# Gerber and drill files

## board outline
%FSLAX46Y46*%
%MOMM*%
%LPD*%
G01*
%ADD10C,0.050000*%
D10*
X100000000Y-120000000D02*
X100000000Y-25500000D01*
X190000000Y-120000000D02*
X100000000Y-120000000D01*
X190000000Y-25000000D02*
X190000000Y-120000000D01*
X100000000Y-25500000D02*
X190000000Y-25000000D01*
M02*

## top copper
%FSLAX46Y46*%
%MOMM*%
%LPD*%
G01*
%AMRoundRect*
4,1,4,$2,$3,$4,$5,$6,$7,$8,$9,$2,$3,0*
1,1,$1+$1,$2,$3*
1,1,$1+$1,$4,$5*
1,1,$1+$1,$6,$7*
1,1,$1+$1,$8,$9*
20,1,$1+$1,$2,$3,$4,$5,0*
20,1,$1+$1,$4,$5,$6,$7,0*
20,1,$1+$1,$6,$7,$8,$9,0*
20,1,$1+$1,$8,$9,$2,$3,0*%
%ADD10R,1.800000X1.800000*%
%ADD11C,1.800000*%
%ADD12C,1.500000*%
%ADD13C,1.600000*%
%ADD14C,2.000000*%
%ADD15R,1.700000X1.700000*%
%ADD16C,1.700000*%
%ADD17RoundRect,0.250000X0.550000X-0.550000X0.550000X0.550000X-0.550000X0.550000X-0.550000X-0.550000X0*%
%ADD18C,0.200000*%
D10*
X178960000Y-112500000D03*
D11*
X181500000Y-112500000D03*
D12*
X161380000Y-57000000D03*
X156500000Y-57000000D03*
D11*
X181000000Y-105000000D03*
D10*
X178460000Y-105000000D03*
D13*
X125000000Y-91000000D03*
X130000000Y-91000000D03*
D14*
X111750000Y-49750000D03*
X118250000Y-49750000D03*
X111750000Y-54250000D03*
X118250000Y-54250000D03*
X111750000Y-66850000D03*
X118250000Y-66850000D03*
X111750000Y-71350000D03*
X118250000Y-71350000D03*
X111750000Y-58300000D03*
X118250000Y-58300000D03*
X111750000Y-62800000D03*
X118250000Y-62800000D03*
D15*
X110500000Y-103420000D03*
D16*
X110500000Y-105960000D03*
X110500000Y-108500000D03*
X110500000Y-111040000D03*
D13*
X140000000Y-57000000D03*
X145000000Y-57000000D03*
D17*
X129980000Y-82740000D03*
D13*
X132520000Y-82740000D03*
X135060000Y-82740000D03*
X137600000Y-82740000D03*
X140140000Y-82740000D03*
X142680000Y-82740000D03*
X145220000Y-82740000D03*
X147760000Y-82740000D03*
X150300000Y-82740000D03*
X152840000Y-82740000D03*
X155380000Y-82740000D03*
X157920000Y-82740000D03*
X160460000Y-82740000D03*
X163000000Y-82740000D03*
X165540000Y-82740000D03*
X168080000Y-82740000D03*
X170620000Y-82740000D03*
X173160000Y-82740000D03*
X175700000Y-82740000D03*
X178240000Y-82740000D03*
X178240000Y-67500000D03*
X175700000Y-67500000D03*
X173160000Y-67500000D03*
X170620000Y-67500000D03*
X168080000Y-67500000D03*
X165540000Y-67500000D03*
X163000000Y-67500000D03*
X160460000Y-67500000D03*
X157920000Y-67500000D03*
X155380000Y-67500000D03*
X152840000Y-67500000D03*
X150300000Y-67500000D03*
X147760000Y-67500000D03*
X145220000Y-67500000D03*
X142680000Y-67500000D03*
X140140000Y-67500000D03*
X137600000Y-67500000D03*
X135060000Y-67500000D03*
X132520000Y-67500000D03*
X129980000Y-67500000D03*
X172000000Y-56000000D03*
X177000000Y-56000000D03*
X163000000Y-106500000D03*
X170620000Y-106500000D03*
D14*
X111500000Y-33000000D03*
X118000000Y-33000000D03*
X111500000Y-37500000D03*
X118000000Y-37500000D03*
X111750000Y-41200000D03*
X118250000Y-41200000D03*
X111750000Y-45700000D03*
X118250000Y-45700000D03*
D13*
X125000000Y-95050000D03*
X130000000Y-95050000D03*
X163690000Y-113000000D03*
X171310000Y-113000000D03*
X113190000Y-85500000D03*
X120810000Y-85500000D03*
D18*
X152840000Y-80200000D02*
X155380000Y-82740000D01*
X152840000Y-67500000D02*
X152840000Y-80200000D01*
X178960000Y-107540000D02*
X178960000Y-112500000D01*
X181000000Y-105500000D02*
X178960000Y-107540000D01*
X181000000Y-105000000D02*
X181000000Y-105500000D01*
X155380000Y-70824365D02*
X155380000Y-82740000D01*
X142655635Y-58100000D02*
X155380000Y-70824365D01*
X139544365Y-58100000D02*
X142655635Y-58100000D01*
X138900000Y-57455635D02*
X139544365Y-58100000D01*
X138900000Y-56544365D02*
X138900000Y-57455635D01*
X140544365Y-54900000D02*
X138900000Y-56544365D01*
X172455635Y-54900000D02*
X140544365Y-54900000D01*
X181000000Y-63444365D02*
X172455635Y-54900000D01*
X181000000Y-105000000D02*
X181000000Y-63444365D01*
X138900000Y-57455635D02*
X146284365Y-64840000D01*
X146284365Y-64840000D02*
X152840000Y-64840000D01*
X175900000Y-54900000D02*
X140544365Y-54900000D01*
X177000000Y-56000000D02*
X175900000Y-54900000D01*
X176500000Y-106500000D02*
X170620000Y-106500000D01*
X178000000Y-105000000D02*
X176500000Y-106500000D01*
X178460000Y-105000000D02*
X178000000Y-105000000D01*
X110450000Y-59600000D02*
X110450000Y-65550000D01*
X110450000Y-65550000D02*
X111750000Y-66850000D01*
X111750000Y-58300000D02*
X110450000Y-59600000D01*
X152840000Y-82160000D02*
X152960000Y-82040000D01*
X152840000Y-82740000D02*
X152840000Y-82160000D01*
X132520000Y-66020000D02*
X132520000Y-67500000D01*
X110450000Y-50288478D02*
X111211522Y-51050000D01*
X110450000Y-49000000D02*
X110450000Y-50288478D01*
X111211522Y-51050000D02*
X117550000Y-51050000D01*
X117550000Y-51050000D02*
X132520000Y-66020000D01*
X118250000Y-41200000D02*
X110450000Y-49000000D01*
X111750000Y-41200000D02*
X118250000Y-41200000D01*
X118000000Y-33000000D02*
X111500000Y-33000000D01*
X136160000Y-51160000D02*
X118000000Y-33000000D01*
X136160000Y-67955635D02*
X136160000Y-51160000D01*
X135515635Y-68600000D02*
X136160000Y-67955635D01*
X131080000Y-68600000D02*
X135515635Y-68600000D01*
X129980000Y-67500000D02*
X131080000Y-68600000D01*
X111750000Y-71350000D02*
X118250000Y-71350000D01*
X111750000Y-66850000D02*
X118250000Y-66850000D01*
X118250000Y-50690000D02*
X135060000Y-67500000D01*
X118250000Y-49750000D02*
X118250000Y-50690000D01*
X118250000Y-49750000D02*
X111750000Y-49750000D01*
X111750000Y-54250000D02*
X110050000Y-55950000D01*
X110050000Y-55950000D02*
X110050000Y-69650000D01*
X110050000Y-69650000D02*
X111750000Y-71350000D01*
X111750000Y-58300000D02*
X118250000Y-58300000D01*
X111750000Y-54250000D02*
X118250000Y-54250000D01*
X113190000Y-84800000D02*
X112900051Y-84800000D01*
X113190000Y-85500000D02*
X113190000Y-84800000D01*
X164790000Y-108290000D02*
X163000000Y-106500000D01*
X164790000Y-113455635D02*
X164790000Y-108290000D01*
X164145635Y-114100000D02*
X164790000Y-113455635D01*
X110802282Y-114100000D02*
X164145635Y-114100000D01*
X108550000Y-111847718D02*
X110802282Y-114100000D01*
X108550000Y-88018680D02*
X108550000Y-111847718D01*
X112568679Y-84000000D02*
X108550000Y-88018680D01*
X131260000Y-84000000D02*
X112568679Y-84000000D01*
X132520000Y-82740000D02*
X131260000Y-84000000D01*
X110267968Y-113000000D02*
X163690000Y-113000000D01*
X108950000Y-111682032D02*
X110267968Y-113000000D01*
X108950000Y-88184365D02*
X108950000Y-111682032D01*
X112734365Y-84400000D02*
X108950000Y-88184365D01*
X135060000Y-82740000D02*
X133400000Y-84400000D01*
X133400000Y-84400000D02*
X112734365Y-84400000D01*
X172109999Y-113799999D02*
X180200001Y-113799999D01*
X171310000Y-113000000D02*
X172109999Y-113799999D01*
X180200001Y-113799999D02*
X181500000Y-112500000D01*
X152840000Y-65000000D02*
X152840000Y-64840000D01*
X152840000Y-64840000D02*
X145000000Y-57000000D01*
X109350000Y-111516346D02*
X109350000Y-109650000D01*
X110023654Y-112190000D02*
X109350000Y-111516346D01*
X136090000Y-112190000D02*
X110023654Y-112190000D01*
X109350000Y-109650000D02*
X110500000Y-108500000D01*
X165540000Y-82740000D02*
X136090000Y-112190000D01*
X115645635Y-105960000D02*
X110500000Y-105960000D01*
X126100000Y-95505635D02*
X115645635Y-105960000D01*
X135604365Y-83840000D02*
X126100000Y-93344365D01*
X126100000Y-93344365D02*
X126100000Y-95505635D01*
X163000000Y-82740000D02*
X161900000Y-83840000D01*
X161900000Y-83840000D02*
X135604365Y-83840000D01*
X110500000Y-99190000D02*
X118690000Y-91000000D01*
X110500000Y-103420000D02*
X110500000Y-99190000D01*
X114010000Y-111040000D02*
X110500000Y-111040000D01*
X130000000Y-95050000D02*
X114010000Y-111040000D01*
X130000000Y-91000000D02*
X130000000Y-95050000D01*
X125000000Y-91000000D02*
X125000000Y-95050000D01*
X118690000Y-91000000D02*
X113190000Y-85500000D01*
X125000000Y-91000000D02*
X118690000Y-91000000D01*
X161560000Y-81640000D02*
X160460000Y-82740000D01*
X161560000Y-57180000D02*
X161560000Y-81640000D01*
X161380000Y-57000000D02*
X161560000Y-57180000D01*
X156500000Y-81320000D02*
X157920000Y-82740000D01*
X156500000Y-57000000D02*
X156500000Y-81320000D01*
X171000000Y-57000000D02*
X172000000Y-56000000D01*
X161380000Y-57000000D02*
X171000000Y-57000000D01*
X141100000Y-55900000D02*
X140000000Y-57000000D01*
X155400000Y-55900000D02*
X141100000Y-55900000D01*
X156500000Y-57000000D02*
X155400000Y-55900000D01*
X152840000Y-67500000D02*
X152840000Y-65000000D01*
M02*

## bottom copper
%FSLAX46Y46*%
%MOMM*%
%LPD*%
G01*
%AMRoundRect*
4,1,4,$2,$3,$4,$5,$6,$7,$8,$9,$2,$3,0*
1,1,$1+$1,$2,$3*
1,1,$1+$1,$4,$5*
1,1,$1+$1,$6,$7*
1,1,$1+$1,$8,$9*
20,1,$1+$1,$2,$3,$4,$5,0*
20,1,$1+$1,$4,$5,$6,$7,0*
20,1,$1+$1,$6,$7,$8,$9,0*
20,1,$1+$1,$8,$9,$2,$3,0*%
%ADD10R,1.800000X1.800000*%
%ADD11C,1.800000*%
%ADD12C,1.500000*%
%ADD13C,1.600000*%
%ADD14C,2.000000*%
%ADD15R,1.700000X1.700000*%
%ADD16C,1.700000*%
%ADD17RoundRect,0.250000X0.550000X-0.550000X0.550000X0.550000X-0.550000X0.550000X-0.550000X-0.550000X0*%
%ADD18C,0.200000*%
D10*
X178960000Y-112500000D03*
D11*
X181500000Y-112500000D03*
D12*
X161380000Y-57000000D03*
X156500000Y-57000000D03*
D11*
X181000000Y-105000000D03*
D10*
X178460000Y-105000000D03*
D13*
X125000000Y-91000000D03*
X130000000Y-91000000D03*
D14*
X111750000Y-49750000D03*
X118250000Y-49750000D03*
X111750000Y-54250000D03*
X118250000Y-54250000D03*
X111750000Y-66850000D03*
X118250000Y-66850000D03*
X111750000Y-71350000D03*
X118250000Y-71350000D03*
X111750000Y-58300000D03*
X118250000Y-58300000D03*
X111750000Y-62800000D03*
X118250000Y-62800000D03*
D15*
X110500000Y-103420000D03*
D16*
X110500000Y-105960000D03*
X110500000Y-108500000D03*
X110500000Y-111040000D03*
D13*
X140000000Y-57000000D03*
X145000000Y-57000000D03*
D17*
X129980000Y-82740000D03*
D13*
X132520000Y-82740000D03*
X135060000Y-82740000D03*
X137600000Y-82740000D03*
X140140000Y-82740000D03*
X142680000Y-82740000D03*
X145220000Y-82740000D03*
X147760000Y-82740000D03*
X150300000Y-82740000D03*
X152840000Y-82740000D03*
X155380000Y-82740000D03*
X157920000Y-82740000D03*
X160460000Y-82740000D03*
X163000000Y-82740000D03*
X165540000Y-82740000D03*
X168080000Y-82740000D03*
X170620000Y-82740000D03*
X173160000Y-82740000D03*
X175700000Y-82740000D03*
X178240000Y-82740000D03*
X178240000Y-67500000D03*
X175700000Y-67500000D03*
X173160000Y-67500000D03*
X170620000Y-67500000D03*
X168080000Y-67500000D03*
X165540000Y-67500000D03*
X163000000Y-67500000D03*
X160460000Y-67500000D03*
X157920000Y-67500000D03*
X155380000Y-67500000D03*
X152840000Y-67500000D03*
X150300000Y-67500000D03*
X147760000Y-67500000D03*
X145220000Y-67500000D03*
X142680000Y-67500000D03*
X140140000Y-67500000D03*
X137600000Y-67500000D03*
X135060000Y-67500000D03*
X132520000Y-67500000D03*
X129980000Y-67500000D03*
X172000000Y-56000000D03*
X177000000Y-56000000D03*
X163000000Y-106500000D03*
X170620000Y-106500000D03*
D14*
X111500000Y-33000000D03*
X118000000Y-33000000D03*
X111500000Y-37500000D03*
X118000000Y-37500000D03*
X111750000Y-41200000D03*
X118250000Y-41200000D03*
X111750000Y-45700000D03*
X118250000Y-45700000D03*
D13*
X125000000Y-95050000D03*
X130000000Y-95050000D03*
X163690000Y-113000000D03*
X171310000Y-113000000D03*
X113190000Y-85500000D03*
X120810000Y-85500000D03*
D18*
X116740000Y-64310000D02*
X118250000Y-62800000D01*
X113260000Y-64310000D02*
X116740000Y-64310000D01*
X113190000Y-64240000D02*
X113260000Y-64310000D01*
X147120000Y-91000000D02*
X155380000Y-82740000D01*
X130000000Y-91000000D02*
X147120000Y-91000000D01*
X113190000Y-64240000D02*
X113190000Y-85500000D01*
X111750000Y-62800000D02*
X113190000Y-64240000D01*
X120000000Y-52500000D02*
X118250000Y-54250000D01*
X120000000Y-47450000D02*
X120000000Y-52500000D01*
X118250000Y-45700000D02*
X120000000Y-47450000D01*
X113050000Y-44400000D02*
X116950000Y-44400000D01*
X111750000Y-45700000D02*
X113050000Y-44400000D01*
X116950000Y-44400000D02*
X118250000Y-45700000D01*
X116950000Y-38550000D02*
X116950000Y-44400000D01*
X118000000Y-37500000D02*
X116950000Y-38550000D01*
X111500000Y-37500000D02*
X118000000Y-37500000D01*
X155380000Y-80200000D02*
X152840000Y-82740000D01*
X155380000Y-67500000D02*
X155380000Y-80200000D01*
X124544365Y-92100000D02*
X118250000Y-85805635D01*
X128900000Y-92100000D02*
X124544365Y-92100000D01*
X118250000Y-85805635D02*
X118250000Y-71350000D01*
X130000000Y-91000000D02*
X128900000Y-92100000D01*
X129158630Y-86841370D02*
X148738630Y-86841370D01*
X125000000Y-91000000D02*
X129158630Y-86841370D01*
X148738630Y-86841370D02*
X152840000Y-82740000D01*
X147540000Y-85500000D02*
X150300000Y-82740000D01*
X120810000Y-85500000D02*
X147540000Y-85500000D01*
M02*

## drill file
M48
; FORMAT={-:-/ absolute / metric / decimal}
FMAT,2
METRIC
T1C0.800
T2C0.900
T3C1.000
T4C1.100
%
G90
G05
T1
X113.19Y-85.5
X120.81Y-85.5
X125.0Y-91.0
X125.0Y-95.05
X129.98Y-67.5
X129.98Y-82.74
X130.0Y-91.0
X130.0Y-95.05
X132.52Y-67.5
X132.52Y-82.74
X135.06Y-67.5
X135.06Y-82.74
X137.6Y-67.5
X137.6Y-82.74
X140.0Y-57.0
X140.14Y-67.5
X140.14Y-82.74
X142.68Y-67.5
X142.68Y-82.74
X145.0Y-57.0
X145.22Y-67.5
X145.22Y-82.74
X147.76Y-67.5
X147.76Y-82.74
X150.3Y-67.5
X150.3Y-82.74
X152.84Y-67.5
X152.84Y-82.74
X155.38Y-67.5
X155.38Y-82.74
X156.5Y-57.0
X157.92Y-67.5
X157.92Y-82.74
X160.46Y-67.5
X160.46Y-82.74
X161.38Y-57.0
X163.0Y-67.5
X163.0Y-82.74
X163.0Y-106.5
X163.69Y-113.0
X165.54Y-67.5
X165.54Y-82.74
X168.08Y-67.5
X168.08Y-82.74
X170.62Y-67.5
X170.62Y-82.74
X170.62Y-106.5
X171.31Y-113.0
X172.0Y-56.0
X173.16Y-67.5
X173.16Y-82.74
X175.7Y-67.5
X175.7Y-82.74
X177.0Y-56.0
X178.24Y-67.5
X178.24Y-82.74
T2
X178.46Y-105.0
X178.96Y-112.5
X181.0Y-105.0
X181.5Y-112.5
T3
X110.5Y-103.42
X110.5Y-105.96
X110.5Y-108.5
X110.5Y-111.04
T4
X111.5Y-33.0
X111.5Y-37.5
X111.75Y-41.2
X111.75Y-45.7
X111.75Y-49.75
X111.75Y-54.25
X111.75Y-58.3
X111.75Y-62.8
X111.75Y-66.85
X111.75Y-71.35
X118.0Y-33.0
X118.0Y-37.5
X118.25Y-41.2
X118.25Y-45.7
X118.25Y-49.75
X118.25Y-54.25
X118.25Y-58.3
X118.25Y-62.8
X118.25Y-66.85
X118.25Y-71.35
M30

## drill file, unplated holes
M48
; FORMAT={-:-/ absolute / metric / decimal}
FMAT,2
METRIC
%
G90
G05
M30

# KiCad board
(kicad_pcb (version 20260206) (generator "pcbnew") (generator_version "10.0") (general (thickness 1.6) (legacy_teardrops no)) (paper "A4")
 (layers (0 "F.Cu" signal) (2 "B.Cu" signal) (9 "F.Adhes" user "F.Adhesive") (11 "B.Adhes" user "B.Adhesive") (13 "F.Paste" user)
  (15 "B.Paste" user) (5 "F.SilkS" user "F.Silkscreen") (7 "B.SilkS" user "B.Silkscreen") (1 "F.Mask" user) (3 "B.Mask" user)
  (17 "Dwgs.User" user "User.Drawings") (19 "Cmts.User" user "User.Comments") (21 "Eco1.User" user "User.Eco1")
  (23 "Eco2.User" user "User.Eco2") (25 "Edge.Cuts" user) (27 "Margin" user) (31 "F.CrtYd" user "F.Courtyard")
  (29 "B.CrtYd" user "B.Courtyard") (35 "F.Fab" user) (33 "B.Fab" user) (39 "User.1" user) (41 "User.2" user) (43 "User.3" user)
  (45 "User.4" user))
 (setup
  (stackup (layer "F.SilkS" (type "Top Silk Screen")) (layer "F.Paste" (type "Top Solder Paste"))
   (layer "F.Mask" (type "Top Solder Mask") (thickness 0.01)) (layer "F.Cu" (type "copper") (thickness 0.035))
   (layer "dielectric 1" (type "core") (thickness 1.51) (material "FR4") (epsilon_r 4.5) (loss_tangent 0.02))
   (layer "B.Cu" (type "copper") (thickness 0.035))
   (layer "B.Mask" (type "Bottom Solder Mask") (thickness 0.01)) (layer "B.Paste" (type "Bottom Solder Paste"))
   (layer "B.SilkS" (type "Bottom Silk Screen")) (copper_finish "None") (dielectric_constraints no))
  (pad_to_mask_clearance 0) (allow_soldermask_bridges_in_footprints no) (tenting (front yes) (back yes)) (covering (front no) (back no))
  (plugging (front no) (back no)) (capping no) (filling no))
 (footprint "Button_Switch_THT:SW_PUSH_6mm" (layer "F.Cu") (at 111.75 49.75)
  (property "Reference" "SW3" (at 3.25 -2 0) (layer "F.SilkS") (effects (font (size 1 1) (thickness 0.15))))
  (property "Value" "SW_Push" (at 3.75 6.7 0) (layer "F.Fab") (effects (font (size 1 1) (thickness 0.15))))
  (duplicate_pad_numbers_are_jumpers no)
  (pad "1" thru_hole circle (at 0 0 90) (size 2 2) (drill 1.1) (layers "*.Cu" "*.Mask") (remove_unused_layers no) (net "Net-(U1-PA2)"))
  (pad "1" thru_hole circle (at 6.5 0 90) (size 2 2) (drill 1.1) (layers "*.Cu" "*.Mask") (remove_unused_layers no) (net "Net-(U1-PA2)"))
  (pad "2" thru_hole circle (at 0 4.5 90) (size 2 2) (drill 1.1) (layers "*.Cu" "*.Mask") (remove_unused_layers no) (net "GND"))
  (pad "2" thru_hole circle (at 6.5 4.5 90) (size 2 2) (drill 1.1) (layers "*.Cu" "*.Mask") (remove_unused_layers no) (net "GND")))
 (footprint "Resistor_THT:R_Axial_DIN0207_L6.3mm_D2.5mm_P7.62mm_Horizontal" (layer "F.Cu") (at 113.19 85.5)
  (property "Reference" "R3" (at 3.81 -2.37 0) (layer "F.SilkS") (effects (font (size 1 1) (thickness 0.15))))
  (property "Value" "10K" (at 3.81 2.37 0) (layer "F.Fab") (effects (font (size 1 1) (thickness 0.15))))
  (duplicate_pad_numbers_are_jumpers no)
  (pad "1" thru_hole circle (at 0 0) (size 1.6 1.6) (drill 0.8) (layers "*.Cu" "*.Mask") (remove_unused_layers no) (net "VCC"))
  (pad "2" thru_hole circle (at 7.62 0) (size 1.6 1.6) (drill 0.8) (layers "*.Cu" "*.Mask") (remove_unused_layers no)
   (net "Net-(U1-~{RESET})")))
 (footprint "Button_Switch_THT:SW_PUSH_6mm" (layer "F.Cu") (at 111.75 41.2)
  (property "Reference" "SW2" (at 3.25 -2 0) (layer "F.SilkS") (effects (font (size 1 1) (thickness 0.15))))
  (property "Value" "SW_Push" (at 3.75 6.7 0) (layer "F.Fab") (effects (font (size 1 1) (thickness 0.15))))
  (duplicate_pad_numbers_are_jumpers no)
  (pad "1" thru_hole circle (at 0 0 90) (size 2 2) (drill 1.1) (layers "*.Cu" "*.Mask") (remove_unused_layers no) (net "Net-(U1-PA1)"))
  (pad "1" thru_hole circle (at 6.5 0 90) (size 2 2) (drill 1.1) (layers "*.Cu" "*.Mask") (remove_unused_layers no) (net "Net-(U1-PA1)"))
  (pad "2" thru_hole circle (at 0 4.5 90) (size 2 2) (drill 1.1) (layers "*.Cu" "*.Mask") (remove_unused_layers no) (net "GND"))
  (pad "2" thru_hole circle (at 6.5 4.5 90) (size 2 2) (drill 1.1) (layers "*.Cu" "*.Mask") (remove_unused_layers no) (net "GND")))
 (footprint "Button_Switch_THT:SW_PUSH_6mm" (layer "F.Cu") (at 111.75 66.85)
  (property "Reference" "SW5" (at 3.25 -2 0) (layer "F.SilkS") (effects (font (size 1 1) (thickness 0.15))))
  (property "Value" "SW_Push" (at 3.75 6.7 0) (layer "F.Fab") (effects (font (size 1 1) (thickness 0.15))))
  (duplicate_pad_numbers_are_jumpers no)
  (pad "1" thru_hole circle (at 0 0 90) (size 2 2) (drill 1.1) (layers "*.Cu" "*.Mask") (remove_unused_layers no) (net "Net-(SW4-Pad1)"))
  (pad "1" thru_hole circle (at 6.5 0 90) (size 2 2) (drill 1.1) (layers "*.Cu" "*.Mask") (remove_unused_layers no) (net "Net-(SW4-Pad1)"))
  (pad "2" thru_hole circle (at 0 4.5 90) (size 2 2) (drill 1.1) (layers "*.Cu" "*.Mask") (remove_unused_layers no) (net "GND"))
  (pad "2" thru_hole circle (at 6.5 4.5 90) (size 2 2) (drill 1.1) (layers "*.Cu" "*.Mask") (remove_unused_layers no) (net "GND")))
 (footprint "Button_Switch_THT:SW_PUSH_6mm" (layer "F.Cu") (at 111.5 33)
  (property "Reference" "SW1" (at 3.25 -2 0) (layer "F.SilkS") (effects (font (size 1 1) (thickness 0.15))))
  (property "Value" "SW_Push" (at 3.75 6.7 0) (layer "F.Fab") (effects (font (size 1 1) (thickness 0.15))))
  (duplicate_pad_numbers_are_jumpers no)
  (pad "1" thru_hole circle (at 0 0 90) (size 2 2) (drill 1.1) (layers "*.Cu" "*.Mask") (remove_unused_layers no) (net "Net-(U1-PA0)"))
  (pad "1" thru_hole circle (at 6.5 0 90) (size 2 2) (drill 1.1) (layers "*.Cu" "*.Mask") (remove_unused_layers no) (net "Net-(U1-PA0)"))
  (pad "2" thru_hole circle (at 0 4.5 90) (size 2 2) (drill 1.1) (layers "*.Cu" "*.Mask") (remove_unused_layers no) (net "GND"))
  (pad "2" thru_hole circle (at 6.5 4.5 90) (size 2 2) (drill 1.1) (layers "*.Cu" "*.Mask") (remove_unused_layers no) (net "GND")))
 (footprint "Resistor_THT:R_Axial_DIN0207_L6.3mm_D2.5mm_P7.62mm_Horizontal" (layer "F.Cu") (at 163.69 113)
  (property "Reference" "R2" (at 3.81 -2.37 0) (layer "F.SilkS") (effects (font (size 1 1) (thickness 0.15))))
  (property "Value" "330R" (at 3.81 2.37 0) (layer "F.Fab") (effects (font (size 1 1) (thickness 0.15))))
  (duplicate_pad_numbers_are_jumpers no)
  (pad "1" thru_hole circle (at 0 0) (size 1.6 1.6) (drill 0.8) (layers "*.Cu" "*.Mask") (remove_unused_layers no) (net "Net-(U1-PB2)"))
  (pad "2" thru_hole circle (at 7.62 0) (size 1.6 1.6) (drill 0.8) (layers "*.Cu" "*.Mask") (remove_unused_layers no) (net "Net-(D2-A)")))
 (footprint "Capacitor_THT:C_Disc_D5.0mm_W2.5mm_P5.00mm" (layer "F.Cu") (at 125 95.05)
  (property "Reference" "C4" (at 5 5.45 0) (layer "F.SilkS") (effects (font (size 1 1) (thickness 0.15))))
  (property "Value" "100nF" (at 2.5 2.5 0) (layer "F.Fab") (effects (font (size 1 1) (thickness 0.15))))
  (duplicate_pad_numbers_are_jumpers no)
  (pad "1" thru_hole circle (at 0 0) (size 1.6 1.6) (drill 0.8) (layers "*.Cu" "*.Mask") (remove_unused_layers no) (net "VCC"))
  (pad "2" thru_hole circle (at 5 0) (size 1.6 1.6) (drill 0.8) (layers "*.Cu" "*.Mask") (remove_unused_layers no) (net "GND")))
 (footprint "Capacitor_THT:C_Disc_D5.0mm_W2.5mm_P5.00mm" (layer "F.Cu") (at 172 56)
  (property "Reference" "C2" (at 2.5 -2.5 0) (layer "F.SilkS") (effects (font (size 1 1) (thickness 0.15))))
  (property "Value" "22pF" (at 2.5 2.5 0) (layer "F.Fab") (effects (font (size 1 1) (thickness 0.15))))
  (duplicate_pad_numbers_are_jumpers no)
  (pad "1" thru_hole circle (at 0 0) (size 1.6 1.6) (drill 0.8) (layers "*.Cu" "*.Mask") (remove_unused_layers no) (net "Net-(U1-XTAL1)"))
  (pad "2" thru_hole circle (at 5 0) (size 1.6 1.6) (drill 0.8) (layers "*.Cu" "*.Mask") (remove_unused_layers no) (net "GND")))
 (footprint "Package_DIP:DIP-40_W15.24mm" (layer "F.Cu") (at 129.98 82.74 90)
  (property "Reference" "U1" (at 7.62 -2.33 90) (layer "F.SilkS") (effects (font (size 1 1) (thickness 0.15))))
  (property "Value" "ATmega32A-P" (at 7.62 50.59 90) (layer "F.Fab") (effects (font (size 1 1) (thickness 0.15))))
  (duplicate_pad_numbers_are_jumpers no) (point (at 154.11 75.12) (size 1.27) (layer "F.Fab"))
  (pad "1" thru_hole roundrect (at 0 0 90) (size 1.6 1.6) (drill 0.8) (layers "*.Cu" "*.Mask") (remove_unused_layers no)
   (roundrect_rratio 0.15625) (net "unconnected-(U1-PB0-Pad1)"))
  (pad "2" thru_hole circle (at 0 2.54 90) (size 1.6 1.6) (drill 0.8) (layers "*.Cu" "*.Mask") (remove_unused_layers no)
   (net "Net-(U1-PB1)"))
  (pad "3" thru_hole circle (at 0 5.08 90) (size 1.6 1.6) (drill 0.8) (layers "*.Cu" "*.Mask") (remove_unused_layers no)
   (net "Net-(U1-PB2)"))
  (pad "4" thru_hole circle (at 0 7.62 90) (size 1.6 1.6) (drill 0.8) (layers "*.Cu" "*.Mask") (remove_unused_layers no)
   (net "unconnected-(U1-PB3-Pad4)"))
  (pad "5" thru_hole circle (at 0 10.16 90) (size 1.6 1.6) (drill 0.8) (layers "*.Cu" "*.Mask") (remove_unused_layers no)
   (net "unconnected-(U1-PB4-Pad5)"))
  (pad "6" thru_hole circle (at 0 12.7 90) (size 1.6 1.6) (drill 0.8) (layers "*.Cu" "*.Mask") (remove_unused_layers no)
   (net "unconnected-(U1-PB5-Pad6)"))
  (pad "7" thru_hole circle (at 0 15.24 90) (size 1.6 1.6) (drill 0.8) (layers "*.Cu" "*.Mask") (remove_unused_layers no)
   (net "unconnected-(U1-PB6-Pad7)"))
  (pad "8" thru_hole circle (at 0 17.78 90) (size 1.6 1.6) (drill 0.8) (layers "*.Cu" "*.Mask") (remove_unused_layers no)
   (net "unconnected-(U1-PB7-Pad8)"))
  (pad "9" thru_hole circle (at 0 20.32 90) (size 1.6 1.6) (drill 0.8) (layers "*.Cu" "*.Mask") (remove_unused_layers no)
   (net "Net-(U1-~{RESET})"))
  (pad "10" thru_hole circle (at 0 22.86 90) (size 1.6 1.6) (drill 0.8) (layers "*.Cu" "*.Mask") (remove_unused_layers no) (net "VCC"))
  (pad "11" thru_hole circle (at 0 25.4 90) (size 1.6 1.6) (drill 0.8) (layers "*.Cu" "*.Mask") (remove_unused_layers no) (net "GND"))
  (pad "12" thru_hole circle (at 0 27.94 90) (size 1.6 1.6) (drill 0.8) (layers "*.Cu" "*.Mask") (remove_unused_layers no)
   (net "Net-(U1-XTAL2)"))
  (pad "13" thru_hole circle (at 0 30.48 90) (size 1.6 1.6) (drill 0.8) (layers "*.Cu" "*.Mask") (remove_unused_layers no)
   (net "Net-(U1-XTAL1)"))
  (pad "14" thru_hole circle (at 0 33.02 90) (size 1.6 1.6) (drill 0.8) (layers "*.Cu" "*.Mask") (remove_unused_layers no)
   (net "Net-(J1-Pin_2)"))
  (pad "15" thru_hole circle (at 0 35.56 90) (size 1.6 1.6) (drill 0.8) (layers "*.Cu" "*.Mask") (remove_unused_layers no)
   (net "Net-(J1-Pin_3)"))
  (pad "16" thru_hole circle (at 0 38.1 90) (size 1.6 1.6) (drill 0.8) (layers "*.Cu" "*.Mask") (remove_unused_layers no)
   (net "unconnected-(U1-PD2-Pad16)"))
  (pad "17" thru_hole circle (at 0 40.64 90) (size 1.6 1.6) (drill 0.8) (layers "*.Cu" "*.Mask") (remove_unused_layers no)
   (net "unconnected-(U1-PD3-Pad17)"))
  (pad "18" thru_hole circle (at 0 43.18 90) (size 1.6 1.6) (drill 0.8) (layers "*.Cu" "*.Mask") (remove_unused_layers no)
   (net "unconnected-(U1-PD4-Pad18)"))
  (pad "19" thru_hole circle (at 0 45.72 90) (size 1.6 1.6) (drill 0.8) (layers "*.Cu" "*.Mask") (remove_unused_layers no)
   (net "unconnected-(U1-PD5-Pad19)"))
  (pad "20" thru_hole circle (at 0 48.26 90) (size 1.6 1.6) (drill 0.8) (layers "*.Cu" "*.Mask") (remove_unused_layers no)
   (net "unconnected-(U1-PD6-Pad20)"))
  (pad "21" thru_hole circle (at 15.24 48.26 90) (size 1.6 1.6) (drill 0.8) (layers "*.Cu" "*.Mask") (remove_unused_layers no)
   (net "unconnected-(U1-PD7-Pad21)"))
  (pad "22" thru_hole circle (at 15.24 45.72 90) (size 1.6 1.6) (drill 0.8) (layers "*.Cu" "*.Mask") (remove_unused_layers no)
   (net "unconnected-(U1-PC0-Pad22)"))
  (pad "23" thru_hole circle (at 15.24 43.18 90) (size 1.6 1.6) (drill 0.8) (layers "*.Cu" "*.Mask") (remove_unused_layers no)
   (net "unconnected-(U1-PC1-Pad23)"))
  (pad "24" thru_hole circle (at 15.24 40.64 90) (size 1.6 1.6) (drill 0.8) (layers "*.Cu" "*.Mask") (remove_unused_layers no)
   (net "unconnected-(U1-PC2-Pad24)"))
  (pad "25" thru_hole circle (at 15.24 38.1 90) (size 1.6 1.6) (drill 0.8) (layers "*.Cu" "*.Mask") (remove_unused_layers no)
   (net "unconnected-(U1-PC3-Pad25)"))
  (pad "26" thru_hole circle (at 15.24 35.56 90) (size 1.6 1.6) (drill 0.8) (layers "*.Cu" "*.Mask") (remove_unused_layers no)
   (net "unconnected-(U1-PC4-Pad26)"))
  (pad "27" thru_hole circle (at 15.24 33.02 90) (size 1.6 1.6) (drill 0.8) (layers "*.Cu" "*.Mask") (remove_unused_layers no)
   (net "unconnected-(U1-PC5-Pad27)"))
  (pad "28" thru_hole circle (at 15.24 30.48 90) (size 1.6 1.6) (drill 0.8) (layers "*.Cu" "*.Mask") (remove_unused_layers no)
   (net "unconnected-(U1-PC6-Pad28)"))
  (pad "29" thru_hole circle (at 15.24 27.94 90) (size 1.6 1.6) (drill 0.8) (layers "*.Cu" "*.Mask") (remove_unused_layers no)
   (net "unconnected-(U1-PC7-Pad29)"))
  (pad "30" thru_hole circle (at 15.24 25.4 90) (size 1.6 1.6) (drill 0.8) (layers "*.Cu" "*.Mask") (remove_unused_layers no) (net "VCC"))
  (pad "31" thru_hole circle (at 15.24 22.86 90) (size 1.6 1.6) (drill 0.8) (layers "*.Cu" "*.Mask") (remove_unused_layers no) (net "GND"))
  (pad "32" thru_hole circle (at 15.24 20.32 90) (size 1.6 1.6) (drill 0.8) (layers "*.Cu" "*.Mask") (remove_unused_layers no)
   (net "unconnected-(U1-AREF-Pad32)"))
  (pad "33" thru_hole circle (at 15.24 17.78 90) (size 1.6 1.6) (drill 0.8) (layers "*.Cu" "*.Mask") (remove_unused_layers no)
   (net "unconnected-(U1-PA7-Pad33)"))
  (pad "34" thru_hole circle (at 15.24 15.24 90) (size 1.6 1.6) (drill 0.8) (layers "*.Cu" "*.Mask") (remove_unused_layers no)
   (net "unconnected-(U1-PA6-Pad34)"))
  (pad "35" thru_hole circle (at 15.24 12.7 90) (size 1.6 1.6) (drill 0.8) (layers "*.Cu" "*.Mask") (remove_unused_layers no)
   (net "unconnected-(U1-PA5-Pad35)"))
  (pad "36" thru_hole circle (at 15.24 10.16 90) (size 1.6 1.6) (drill 0.8) (layers "*.Cu" "*.Mask") (remove_unused_layers no)
   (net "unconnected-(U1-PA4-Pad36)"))
  (pad "37" thru_hole circle (at 15.24 7.62 90) (size 1.6 1.6) (drill 0.8) (layers "*.Cu" "*.Mask") (remove_unused_layers no)
   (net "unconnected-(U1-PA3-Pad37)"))
  (pad "38" thru_hole circle (at 15.24 5.08 90) (size 1.6 1.6) (drill 0.8) (layers "*.Cu" "*.Mask") (remove_unused_layers no)
   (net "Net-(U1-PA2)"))
  (pad "39" thru_hole circle (at 15.24 2.54 90) (size 1.6 1.6) (drill 0.8) (layers "*.Cu" "*.Mask") (remove_unused_layers no)
   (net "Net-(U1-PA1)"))
  (pad "40" thru_hole circle (at 15.24 0 90) (size 1.6 1.6) (drill 0.8) (layers "*.Cu" "*.Mask") (remove_unused_layers no)
   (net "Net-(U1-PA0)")))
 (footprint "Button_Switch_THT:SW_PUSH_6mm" (layer "F.Cu") (at 111.75 58.3)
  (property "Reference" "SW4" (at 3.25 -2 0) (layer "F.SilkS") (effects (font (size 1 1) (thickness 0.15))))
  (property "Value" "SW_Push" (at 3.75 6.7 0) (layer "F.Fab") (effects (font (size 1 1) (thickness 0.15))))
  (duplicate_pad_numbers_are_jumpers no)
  (pad "1" thru_hole circle (at 0 0 90) (size 2 2) (drill 1.1) (layers "*.Cu" "*.Mask") (remove_unused_layers no) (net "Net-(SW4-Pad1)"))
  (pad "1" thru_hole circle (at 6.5 0 90) (size 2 2) (drill 1.1) (layers "*.Cu" "*.Mask") (remove_unused_layers no) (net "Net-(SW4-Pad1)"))
  (pad "2" thru_hole circle (at 0 4.5 90) (size 2 2) (drill 1.1) (layers "*.Cu" "*.Mask") (remove_unused_layers no) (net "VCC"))
  (pad "2" thru_hole circle (at 6.5 4.5 90) (size 2 2) (drill 1.1) (layers "*.Cu" "*.Mask") (remove_unused_layers no) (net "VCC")))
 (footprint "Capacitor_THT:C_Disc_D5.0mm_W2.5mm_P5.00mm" (layer "F.Cu") (at 125 91)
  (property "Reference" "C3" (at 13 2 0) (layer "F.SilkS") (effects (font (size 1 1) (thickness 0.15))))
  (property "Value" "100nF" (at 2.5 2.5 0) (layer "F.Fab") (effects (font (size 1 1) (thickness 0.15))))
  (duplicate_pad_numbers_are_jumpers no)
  (pad "1" thru_hole circle (at 0 0) (size 1.6 1.6) (drill 0.8) (layers "*.Cu" "*.Mask") (remove_unused_layers no) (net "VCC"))
  (pad "2" thru_hole circle (at 5 0) (size 1.6 1.6) (drill 0.8) (layers "*.Cu" "*.Mask") (remove_unused_layers no) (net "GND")))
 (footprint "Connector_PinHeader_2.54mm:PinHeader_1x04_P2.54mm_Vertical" (layer "F.Cu") (at 110.5 103.42)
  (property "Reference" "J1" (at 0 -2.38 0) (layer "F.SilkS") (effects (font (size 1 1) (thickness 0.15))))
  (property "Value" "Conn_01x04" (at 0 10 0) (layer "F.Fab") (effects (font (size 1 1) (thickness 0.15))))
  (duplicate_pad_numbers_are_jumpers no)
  (pad "1" thru_hole rect (at 0 0) (size 1.7 1.7) (drill 1) (layers "*.Cu" "*.Mask") (remove_unused_layers no) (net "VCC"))
  (pad "2" thru_hole circle (at 0 2.54) (size 1.7 1.7) (drill 1) (layers "*.Cu" "*.Mask") (remove_unused_layers no) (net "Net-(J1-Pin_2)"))
  (pad "3" thru_hole circle (at 0 5.08) (size 1.7 1.7) (drill 1) (layers "*.Cu" "*.Mask") (remove_unused_layers no) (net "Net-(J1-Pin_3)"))
  (pad "4" thru_hole circle (at 0 7.62) (size 1.7 1.7) (drill 1) (layers "*.Cu" "*.Mask") (remove_unused_layers no) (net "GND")))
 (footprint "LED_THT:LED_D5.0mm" (layer "F.Cu") (at 178.96 112.5)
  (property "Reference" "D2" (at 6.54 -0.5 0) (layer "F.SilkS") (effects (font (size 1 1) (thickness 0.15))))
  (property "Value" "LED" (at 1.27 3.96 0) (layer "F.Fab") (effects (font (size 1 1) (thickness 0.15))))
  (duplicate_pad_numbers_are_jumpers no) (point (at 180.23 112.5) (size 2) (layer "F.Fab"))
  (pad "1" thru_hole rect (at 0 0) (size 1.8 1.8) (drill 0.9) (layers "*.Cu" "*.Mask") (remove_unused_layers no) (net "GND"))
  (pad "2" thru_hole circle (at 2.54 0) (size 1.8 1.8) (drill 0.9) (layers "*.Cu" "*.Mask") (remove_unused_layers no) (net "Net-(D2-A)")))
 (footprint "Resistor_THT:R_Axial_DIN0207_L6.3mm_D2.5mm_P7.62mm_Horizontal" (layer "F.Cu") (at 163 106.5)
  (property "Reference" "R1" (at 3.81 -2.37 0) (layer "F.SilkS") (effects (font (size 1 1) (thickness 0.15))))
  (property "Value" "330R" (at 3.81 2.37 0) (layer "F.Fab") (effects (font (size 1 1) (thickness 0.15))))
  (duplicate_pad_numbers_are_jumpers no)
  (pad "1" thru_hole circle (at 0 0) (size 1.6 1.6) (drill 0.8) (layers "*.Cu" "*.Mask") (remove_unused_layers no) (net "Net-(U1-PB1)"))
  (pad "2" thru_hole circle (at 7.62 0) (size 1.6 1.6) (drill 0.8) (layers "*.Cu" "*.Mask") (remove_unused_layers no) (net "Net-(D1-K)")))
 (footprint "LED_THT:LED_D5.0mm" (layer "F.Cu") (at 178.46 105)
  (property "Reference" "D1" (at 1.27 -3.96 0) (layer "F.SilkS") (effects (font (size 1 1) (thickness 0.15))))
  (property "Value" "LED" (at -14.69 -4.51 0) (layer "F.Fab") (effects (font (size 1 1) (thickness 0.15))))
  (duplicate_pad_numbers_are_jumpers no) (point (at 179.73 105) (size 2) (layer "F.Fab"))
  (pad "1" thru_hole rect (at 0 0) (size 1.8 1.8) (drill 0.9) (layers "*.Cu" "*.Mask") (remove_unused_layers no) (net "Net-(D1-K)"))
  (pad "2" thru_hole circle (at 2.54 0) (size 1.8 1.8) (drill 0.9) (layers "*.Cu" "*.Mask") (remove_unused_layers no) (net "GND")))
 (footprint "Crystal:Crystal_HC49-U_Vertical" (layer "F.Cu") (at 156.5 57)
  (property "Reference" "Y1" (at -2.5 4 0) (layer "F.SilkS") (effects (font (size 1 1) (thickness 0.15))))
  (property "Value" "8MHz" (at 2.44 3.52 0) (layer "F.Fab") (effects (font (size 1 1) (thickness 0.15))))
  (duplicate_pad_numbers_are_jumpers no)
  (pad "1" thru_hole circle (at 0 0) (size 1.5 1.5) (drill 0.8) (layers "*.Cu" "*.Mask") (remove_unused_layers no) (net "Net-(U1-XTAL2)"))
  (pad "2" thru_hole circle (at 4.88 0) (size 1.5 1.5) (drill 0.8) (layers "*.Cu" "*.Mask") (remove_unused_layers no) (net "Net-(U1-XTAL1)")))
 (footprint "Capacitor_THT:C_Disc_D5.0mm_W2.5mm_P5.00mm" (layer "F.Cu") (at 140 57)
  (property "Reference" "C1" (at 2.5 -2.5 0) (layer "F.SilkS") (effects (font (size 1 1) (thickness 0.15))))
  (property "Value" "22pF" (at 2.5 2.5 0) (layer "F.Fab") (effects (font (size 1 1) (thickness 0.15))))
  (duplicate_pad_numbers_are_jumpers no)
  (pad "1" thru_hole circle (at 0 0) (size 1.6 1.6) (drill 0.8) (layers "*.Cu" "*.Mask") (remove_unused_layers no) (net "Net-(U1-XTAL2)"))
  (pad "2" thru_hole circle (at 5 0) (size 1.6 1.6) (drill 0.8) (layers "*.Cu" "*.Mask") (remove_unused_layers no) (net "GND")))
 (gr_line (start 100 25.5) (end 190 25) (stroke (width 0.05) (type default)) (layer "Edge.Cuts"))
 (gr_line (start 100 120) (end 100 25.5) (stroke (width 0.05) (type default)) (layer "Edge.Cuts"))
 (gr_line (start 190 25) (end 190 120) (stroke (width 0.05) (type default)) (layer "Edge.Cuts"))
 (gr_line (start 190 120) (end 100 120) (stroke (width 0.05) (type default)) (layer "Edge.Cuts"))
 (segment (start 110.05 55.95) (end 110.05 69.65) (width 0.2) (layer "F.Cu") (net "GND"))
 (segment (start 181 105.5) (end 178.96 107.54) (width 0.2) (layer "F.Cu") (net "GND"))
 (segment (start 138.9 57.455635) (end 139.544365 58.1) (width 0.2) (layer "F.Cu") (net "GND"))
 (segment (start 142.655635 58.1) (end 155.38 70.824365) (width 0.2) (layer "F.Cu") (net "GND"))
 (segment (start 152.84 80.2) (end 155.38 82.74) (width 0.2) (layer "F.Cu") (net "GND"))
 (segment (start 138.9 57.455635) (end 146.284365 64.84) (width 0.2) (layer "F.Cu") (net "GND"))
 (segment (start 175.9 54.9) (end 140.544365 54.9) (width 0.2) (layer "F.Cu") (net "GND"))
 (segment (start 177 56) (end 175.9 54.9) (width 0.2) (layer "F.Cu") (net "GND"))
 (segment (start 152.84 65) (end 152.84 64.84) (width 0.2) (layer "F.Cu") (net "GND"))
 (segment (start 111.75 54.25) (end 118.25 54.25) (width 0.2) (layer "F.Cu") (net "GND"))
 (segment (start 152.84 67.5) (end 152.84 65) (width 0.2) (layer "F.Cu") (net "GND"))
 (segment (start 146.284365 64.84) (end 152.84 64.84) (width 0.2) (layer "F.Cu") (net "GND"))
 (segment (start 110.05 69.65) (end 111.75 71.35) (width 0.2) (layer "F.Cu") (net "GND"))
 (segment (start 152.84 64.84) (end 145 57) (width 0.2) (layer "F.Cu") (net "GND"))
 (segment (start 178.96 107.54) (end 178.96 112.5) (width 0.2) (layer "F.Cu") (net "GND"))
 (segment (start 140.544365 54.9) (end 138.9 56.544365) (width 0.2) (layer "F.Cu") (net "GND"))
 (segment (start 114.01 111.04) (end 110.5 111.04) (width 0.2) (layer "F.Cu") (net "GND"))
 (segment (start 138.9 56.544365) (end 138.9 57.455635) (width 0.2) (layer "F.Cu") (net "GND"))
 (segment (start 111.75 71.35) (end 118.25 71.35) (width 0.2) (layer "F.Cu") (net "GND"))
 (segment (start 181 105) (end 181 63.444365) (width 0.2) (layer "F.Cu") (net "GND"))
 (segment (start 181 105) (end 181 105.5) (width 0.2) (layer "F.Cu") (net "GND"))
 (segment (start 130 91) (end 130 95.05) (width 0.2) (layer "F.Cu") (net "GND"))
 (segment (start 172.455635 54.9) (end 140.544365 54.9) (width 0.2) (layer "F.Cu") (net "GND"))
 (segment (start 139.544365 58.1) (end 142.655635 58.1) (width 0.2) (layer "F.Cu") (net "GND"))
 (segment (start 155.38 70.824365) (end 155.38 82.74) (width 0.2) (layer "F.Cu") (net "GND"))
 (segment (start 130 95.05) (end 114.01 111.04) (width 0.2) (layer "F.Cu") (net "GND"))
 (segment (start 152.84 67.5) (end 152.84 80.2) (width 0.2) (layer "F.Cu") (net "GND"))
 (segment (start 181 63.444365) (end 172.455635 54.9) (width 0.2) (layer "F.Cu") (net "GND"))
 (segment (start 111.75 54.25) (end 110.05 55.95) (width 0.2) (layer "F.Cu") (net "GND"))
 (segment (start 120 47.45) (end 120 52.5) (width 0.2) (layer "B.Cu") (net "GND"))
 (segment (start 111.75 45.7) (end 113.05 44.4) (width 0.2) (layer "B.Cu") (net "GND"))
 (segment (start 113.05 44.4) (end 116.95 44.4) (width 0.2) (layer "B.Cu") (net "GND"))
 (segment (start 111.5 37.5) (end 118 37.5) (width 0.2) (layer "B.Cu") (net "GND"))
 (segment (start 124.544365 92.1) (end 118.25 85.805635) (width 0.2) (layer "B.Cu") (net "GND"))
 (segment (start 120 52.5) (end 118.25 54.25) (width 0.2) (layer "B.Cu") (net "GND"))
 (segment (start 118.25 85.805635) (end 118.25 71.35) (width 0.2) (layer "B.Cu") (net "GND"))
 (segment (start 116.95 44.4) (end 118.25 45.7) (width 0.2) (layer "B.Cu") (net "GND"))
 (segment (start 118 37.5) (end 116.95 38.55) (width 0.2) (layer "B.Cu") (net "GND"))
 (segment (start 130 91) (end 128.9 92.1) (width 0.2) (layer "B.Cu") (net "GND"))
 (segment (start 130 91) (end 147.12 91) (width 0.2) (layer "B.Cu") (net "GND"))
 (segment (start 116.95 38.55) (end 116.95 44.4) (width 0.2) (layer "B.Cu") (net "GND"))
 (segment (start 147.12 91) (end 155.38 82.74) (width 0.2) (layer "B.Cu") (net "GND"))
 (segment (start 128.9 92.1) (end 124.544365 92.1) (width 0.2) (layer "B.Cu") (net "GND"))
 (segment (start 118.25 45.7) (end 120 47.45) (width 0.2) (layer "B.Cu") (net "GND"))
 (segment (start 156.5 81.32) (end 157.92 82.74) (width 0.2) (layer "F.Cu") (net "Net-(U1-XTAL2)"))
 (segment (start 156.5 57) (end 156.5 81.32) (width 0.2) (layer "F.Cu") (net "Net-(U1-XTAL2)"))
 (segment (start 141.1 55.9) (end 140 57) (width 0.2) (layer "F.Cu") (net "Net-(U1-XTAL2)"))
 (segment (start 156.5 57) (end 155.4 55.9) (width 0.2) (layer "F.Cu") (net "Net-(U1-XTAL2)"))
 (segment (start 155.4 55.9) (end 141.1 55.9) (width 0.2) (layer "F.Cu") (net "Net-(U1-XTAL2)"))
 (segment (start 161.56 81.64) (end 160.46 82.74) (width 0.2) (layer "F.Cu") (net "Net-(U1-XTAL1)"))
 (segment (start 161.56 57.18) (end 161.56 81.64) (width 0.2) (layer "F.Cu") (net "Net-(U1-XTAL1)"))
 (segment (start 171 57) (end 172 56) (width 0.2) (layer "F.Cu") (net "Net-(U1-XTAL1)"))
 (segment (start 161.38 57) (end 161.56 57.18) (width 0.2) (layer "F.Cu") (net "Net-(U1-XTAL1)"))
 (segment (start 161.38 57) (end 171 57) (width 0.2) (layer "F.Cu") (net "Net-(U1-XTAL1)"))
 (segment (start 110.5 99.19) (end 118.69 91) (width 0.2) (layer "F.Cu") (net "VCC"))
 (segment (start 152.84 82.16) (end 152.96 82.04) (width 0.2) (layer "F.Cu") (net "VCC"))
 (segment (start 118.69 91) (end 113.19 85.5) (width 0.2) (layer "F.Cu") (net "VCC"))
 (segment (start 113.19 84.8) (end 112.900051 84.8) (width 0.2) (layer "F.Cu") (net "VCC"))
 (segment (start 152.84 82.74) (end 152.84 82.16) (width 0.2) (layer "F.Cu") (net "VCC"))
 (segment (start 113.19 85.5) (end 113.19 84.8) (width 0.2) (layer "F.Cu") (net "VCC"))
 (segment (start 110.5 103.42) (end 110.5 99.19) (width 0.2) (layer "F.Cu") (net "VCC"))
 (segment (start 125 91) (end 125 95.05) (width 0.2) (layer "F.Cu") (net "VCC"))
 (segment (start 125 91) (end 118.69 91) (width 0.2) (layer "F.Cu") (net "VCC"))
 (segment (start 125 91) (end 129.15863 86.84137) (width 0.2) (layer "B.Cu") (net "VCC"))
 (segment (start 111.75 62.8) (end 113.19 64.24) (width 0.2) (layer "B.Cu") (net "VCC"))
 (segment (start 155.38 80.2) (end 152.84 82.74) (width 0.2) (layer "B.Cu") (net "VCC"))
 (segment (start 116.74 64.31) (end 118.25 62.8) (width 0.2) (layer "B.Cu") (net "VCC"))
 (segment (start 113.19 64.24) (end 113.26 64.31) (width 0.2) (layer "B.Cu") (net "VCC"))
 (segment (start 113.26 64.31) (end 116.74 64.31) (width 0.2) (layer "B.Cu") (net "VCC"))
 (segment (start 148.73863 86.84137) (end 152.84 82.74) (width 0.2) (layer "B.Cu") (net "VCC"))
 (segment (start 129.15863 86.84137) (end 148.73863 86.84137) (width 0.2) (layer "B.Cu") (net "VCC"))
 (segment (start 113.19 64.24) (end 113.19 85.5) (width 0.2) (layer "B.Cu") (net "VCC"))
 (segment (start 155.38 67.5) (end 155.38 80.2) (width 0.2) (layer "B.Cu") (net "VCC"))
 (segment (start 178.46 105) (end 178 105) (width 0.2) (layer "F.Cu") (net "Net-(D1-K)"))
 (segment (start 178 105) (end 176.5 106.5) (width 0.2) (layer "F.Cu") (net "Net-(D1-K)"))
 (segment (start 176.5 106.5) (end 170.62 106.5) (width 0.2) (layer "F.Cu") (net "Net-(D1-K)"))
 (segment (start 171.31 113) (end 172.109999 113.799999) (width 0.2) (layer "F.Cu") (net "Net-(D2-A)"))
 (segment (start 180.200001 113.799999) (end 181.5 112.5) (width 0.2) (layer "F.Cu") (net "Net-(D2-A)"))
 (segment (start 172.109999 113.799999) (end 180.200001 113.799999) (width 0.2) (layer "F.Cu") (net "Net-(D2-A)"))
 (segment (start 115.645635 105.96) (end 110.5 105.96) (width 0.2) (layer "F.Cu") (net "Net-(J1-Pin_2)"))
 (segment (start 161.9 83.84) (end 135.604365 83.84) (width 0.2) (layer "F.Cu") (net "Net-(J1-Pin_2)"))
 (segment (start 163 82.74) (end 161.9 83.84) (width 0.2) (layer "F.Cu") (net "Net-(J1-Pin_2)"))
 (segment (start 135.604365 83.84) (end 126.1 93.344365) (width 0.2) (layer "F.Cu") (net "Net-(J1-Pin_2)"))
 (segment (start 126.1 95.505635) (end 115.645635 105.96) (width 0.2) (layer "F.Cu") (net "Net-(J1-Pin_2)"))
 (segment (start 126.1 93.344365) (end 126.1 95.505635) (width 0.2) (layer "F.Cu") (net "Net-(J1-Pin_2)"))
 (segment (start 165.54 82.74) (end 136.09 112.19) (width 0.2) (layer "F.Cu") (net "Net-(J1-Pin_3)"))
 (segment (start 136.09 112.19) (end 110.023654 112.19) (width 0.2) (layer "F.Cu") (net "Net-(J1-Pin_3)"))
 (segment (start 110.023654 112.19) (end 109.35 111.516346) (width 0.2) (layer "F.Cu") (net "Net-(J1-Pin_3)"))
 (segment (start 109.35 109.65) (end 110.5 108.5) (width 0.2) (layer "F.Cu") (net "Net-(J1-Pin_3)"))
 (segment (start 109.35 111.516346) (end 109.35 109.65) (width 0.2) (layer "F.Cu") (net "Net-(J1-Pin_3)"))
 (segment (start 131.26 84) (end 112.568679 84) (width 0.2) (layer "F.Cu") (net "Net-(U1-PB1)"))
 (segment (start 164.145635 114.1) (end 164.79 113.455635) (width 0.2) (layer "F.Cu") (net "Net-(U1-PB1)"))
 (segment (start 112.568679 84) (end 108.55 88.01868) (width 0.2) (layer "F.Cu") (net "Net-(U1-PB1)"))
 (segment (start 110.802282 114.1) (end 164.145635 114.1) (width 0.2) (layer "F.Cu") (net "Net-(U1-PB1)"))
 (segment (start 132.52 82.74) (end 131.26 84) (width 0.2) (layer "F.Cu") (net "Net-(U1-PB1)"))
 (segment (start 164.79 108.29) (end 163 106.5) (width 0.2) (layer "F.Cu") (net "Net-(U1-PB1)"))
 (segment (start 164.79 113.455635) (end 164.79 108.29) (width 0.2) (layer "F.Cu") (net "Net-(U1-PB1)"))
 (segment (start 108.55 88.01868) (end 108.55 111.847718) (width 0.2) (layer "F.Cu") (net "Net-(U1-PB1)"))
 (segment (start 108.55 111.847718) (end 110.802282 114.1) (width 0.2) (layer "F.Cu") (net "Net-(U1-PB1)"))
 (segment (start 112.734365 84.4) (end 108.95 88.184365) (width 0.2) (layer "F.Cu") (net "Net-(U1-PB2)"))
 (segment (start 110.267968 113) (end 163.69 113) (width 0.2) (layer "F.Cu") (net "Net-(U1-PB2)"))
 (segment (start 135.06 82.74) (end 133.4 84.4) (width 0.2) (layer "F.Cu") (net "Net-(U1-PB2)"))
 (segment (start 133.4 84.4) (end 112.734365 84.4) (width 0.2) (layer "F.Cu") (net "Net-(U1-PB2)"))
 (segment (start 108.95 111.682032) (end 110.267968 113) (width 0.2) (layer "F.Cu") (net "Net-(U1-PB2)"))
 (segment (start 108.95 88.184365) (end 108.95 111.682032) (width 0.2) (layer "F.Cu") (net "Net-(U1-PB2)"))
 (segment (start 120.81 85.5) (end 147.54 85.5) (width 0.2) (layer "B.Cu") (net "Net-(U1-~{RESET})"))
 (segment (start 147.54 85.5) (end 150.3 82.74) (width 0.2) (layer "B.Cu") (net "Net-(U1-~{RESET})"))
 (segment (start 131.08 68.6) (end 135.515635 68.6) (width 0.2) (layer "F.Cu") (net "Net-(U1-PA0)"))
 (segment (start 135.515635 68.6) (end 136.16 67.955635) (width 0.2) (layer "F.Cu") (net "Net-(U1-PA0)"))
 (segment (start 129.98 67.5) (end 131.08 68.6) (width 0.2) (layer "F.Cu") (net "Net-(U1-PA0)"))
 (segment (start 136.16 67.955635) (end 136.16 51.16) (width 0.2) (layer "F.Cu") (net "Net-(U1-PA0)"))
 (segment (start 118 33) (end 111.5 33) (width 0.2) (layer "F.Cu") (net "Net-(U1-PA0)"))
 (segment (start 136.16 51.16) (end 118 33) (width 0.2) (layer "F.Cu") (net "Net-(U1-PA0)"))
 (segment (start 132.52 66.02) (end 132.52 67.5) (width 0.2) (layer "F.Cu") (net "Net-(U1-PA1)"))
 (segment (start 117.55 51.05) (end 132.52 66.02) (width 0.2) (layer "F.Cu") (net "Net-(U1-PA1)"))
 (segment (start 111.211522 51.05) (end 117.55 51.05) (width 0.2) (layer "F.Cu") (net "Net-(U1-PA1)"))
 (segment (start 110.45 50.288478) (end 111.211522 51.05) (width 0.2) (layer "F.Cu") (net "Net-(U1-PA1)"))
 (segment (start 118.25 41.2) (end 110.45 49) (width 0.2) (layer "F.Cu") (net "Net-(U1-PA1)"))
 (segment (start 111.75 41.2) (end 118.25 41.2) (width 0.2) (layer "F.Cu") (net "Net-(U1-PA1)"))
 (segment (start 110.45 49) (end 110.45 50.288478) (width 0.2) (layer "F.Cu") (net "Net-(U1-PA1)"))
 (segment (start 118.25 49.75) (end 118.25 50.69) (width 0.2) (layer "F.Cu") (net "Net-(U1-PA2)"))
 (segment (start 118.25 50.69) (end 135.06 67.5) (width 0.2) (layer "F.Cu") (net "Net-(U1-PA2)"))
 (segment (start 118.25 49.75) (end 111.75 49.75) (width 0.2) (layer "F.Cu") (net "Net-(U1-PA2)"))
 (segment (start 110.45 59.6) (end 110.45 65.55) (width 0.2) (layer "F.Cu") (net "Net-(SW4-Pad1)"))
 (segment (start 111.75 66.85) (end 118.25 66.85) (width 0.2) (layer "F.Cu") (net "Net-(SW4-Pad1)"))
 (segment (start 111.75 58.3) (end 118.25 58.3) (width 0.2) (layer "F.Cu") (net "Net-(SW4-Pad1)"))
 (segment (start 111.75 58.3) (end 110.45 59.6) (width 0.2) (layer "F.Cu") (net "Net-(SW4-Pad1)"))
 (segment (start 110.45 65.55) (end 111.75 66.85) (width 0.2) (layer "F.Cu") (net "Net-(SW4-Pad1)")))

